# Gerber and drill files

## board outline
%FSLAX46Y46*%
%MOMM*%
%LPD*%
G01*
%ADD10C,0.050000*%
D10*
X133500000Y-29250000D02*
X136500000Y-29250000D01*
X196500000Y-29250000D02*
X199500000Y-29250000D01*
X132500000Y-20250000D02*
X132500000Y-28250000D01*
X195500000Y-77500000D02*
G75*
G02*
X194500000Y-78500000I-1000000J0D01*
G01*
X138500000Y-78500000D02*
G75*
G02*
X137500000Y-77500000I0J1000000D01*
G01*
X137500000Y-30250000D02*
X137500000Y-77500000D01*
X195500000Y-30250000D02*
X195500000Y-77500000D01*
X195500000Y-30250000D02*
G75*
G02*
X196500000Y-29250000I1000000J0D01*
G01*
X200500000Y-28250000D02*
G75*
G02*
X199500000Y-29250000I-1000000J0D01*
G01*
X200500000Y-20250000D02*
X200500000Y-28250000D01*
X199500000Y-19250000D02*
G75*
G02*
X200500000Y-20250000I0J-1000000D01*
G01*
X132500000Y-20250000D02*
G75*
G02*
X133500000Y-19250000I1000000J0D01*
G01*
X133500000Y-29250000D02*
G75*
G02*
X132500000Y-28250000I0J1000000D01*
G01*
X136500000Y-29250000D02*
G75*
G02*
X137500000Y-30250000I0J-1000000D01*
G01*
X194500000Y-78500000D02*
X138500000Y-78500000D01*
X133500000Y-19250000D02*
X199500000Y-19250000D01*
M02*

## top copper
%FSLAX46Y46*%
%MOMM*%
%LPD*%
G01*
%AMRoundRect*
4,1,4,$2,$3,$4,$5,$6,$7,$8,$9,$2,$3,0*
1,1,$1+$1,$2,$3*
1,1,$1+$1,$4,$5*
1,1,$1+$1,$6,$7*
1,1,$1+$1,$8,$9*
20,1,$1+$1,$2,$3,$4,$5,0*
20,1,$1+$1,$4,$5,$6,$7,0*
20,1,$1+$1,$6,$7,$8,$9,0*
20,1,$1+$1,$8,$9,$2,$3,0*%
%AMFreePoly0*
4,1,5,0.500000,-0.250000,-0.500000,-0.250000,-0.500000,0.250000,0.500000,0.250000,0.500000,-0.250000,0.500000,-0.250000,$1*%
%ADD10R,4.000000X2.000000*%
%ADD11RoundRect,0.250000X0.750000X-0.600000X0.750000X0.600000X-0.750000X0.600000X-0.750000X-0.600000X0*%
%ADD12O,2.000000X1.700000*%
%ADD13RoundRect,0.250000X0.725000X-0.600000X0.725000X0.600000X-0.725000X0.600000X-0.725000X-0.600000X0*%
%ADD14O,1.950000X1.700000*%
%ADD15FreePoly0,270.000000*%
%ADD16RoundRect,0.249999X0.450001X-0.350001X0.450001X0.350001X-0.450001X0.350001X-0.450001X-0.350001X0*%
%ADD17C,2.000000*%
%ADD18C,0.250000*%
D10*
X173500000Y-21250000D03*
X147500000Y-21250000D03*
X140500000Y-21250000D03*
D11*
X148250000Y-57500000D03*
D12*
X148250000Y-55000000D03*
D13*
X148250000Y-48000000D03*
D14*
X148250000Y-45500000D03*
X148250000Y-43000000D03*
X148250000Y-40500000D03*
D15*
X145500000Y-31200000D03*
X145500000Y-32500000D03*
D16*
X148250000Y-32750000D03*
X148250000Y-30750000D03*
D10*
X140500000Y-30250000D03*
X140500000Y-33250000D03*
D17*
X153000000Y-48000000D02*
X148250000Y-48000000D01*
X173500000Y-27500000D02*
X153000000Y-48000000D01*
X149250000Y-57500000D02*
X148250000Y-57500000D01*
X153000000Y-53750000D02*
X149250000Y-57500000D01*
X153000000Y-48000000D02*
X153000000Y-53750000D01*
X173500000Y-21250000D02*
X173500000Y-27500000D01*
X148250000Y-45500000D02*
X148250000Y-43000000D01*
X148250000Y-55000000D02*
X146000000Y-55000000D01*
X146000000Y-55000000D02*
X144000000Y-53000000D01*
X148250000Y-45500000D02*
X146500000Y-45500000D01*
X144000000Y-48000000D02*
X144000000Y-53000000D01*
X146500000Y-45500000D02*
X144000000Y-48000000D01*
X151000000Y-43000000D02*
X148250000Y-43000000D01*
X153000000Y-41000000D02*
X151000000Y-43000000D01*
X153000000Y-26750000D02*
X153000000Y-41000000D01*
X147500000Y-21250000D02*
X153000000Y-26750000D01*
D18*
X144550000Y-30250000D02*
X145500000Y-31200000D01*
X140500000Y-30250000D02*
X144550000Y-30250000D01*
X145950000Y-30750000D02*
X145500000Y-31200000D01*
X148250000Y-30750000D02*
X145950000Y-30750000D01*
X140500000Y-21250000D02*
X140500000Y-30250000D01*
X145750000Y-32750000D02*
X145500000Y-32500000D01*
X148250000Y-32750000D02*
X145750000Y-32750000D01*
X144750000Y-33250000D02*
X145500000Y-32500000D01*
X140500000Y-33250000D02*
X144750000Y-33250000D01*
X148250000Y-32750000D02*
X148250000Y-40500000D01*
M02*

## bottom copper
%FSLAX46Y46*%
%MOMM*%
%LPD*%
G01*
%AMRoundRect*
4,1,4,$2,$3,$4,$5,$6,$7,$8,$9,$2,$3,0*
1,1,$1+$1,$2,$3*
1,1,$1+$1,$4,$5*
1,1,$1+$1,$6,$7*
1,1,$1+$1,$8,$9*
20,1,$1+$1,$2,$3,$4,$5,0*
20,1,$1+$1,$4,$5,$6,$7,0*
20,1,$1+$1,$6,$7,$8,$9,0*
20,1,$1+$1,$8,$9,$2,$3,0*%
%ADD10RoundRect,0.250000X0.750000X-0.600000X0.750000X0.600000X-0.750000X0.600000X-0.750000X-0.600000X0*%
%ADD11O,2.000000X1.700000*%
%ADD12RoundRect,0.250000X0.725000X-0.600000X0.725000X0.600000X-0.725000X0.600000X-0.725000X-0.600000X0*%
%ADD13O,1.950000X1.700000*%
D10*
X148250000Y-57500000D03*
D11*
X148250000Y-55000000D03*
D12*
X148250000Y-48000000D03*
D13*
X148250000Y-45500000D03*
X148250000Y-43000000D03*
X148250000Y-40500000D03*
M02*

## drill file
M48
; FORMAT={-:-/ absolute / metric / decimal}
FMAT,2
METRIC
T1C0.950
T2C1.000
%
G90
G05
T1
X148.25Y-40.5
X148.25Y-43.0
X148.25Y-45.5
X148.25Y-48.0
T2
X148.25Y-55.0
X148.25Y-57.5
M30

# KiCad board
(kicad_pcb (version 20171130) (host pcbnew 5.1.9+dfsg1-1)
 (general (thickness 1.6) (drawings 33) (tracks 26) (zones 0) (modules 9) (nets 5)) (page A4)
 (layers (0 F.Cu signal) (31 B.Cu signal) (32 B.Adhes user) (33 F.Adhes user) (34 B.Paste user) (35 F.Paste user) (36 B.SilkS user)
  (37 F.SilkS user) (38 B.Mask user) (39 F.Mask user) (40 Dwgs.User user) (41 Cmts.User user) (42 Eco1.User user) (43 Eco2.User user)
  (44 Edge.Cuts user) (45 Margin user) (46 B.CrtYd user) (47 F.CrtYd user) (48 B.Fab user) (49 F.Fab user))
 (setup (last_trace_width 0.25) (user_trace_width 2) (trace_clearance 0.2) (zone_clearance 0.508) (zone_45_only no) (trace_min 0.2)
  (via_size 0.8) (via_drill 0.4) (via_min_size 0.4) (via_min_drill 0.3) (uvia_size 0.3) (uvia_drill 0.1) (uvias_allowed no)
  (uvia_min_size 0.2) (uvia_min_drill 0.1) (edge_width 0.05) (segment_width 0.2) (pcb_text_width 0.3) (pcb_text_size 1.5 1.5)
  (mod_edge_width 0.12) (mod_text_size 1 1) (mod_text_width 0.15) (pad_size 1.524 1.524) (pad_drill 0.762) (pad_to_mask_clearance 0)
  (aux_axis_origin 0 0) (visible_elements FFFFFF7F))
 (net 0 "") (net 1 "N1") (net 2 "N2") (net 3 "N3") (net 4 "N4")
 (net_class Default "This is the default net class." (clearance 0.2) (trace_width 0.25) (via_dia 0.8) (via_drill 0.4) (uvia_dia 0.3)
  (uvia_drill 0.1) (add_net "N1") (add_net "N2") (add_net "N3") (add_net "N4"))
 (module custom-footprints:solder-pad (layer F.Cu) (at 176.04 21.25 90)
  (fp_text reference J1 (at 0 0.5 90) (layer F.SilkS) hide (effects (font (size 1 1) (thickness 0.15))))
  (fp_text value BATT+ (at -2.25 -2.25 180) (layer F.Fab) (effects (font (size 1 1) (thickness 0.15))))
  (pad 1 smd rect (at 0 -2.54 90) (size 2 4) (layers F.Cu F.Paste F.Mask) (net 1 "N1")))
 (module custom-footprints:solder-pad (layer F.Cu) (at 150.04 21.25 90)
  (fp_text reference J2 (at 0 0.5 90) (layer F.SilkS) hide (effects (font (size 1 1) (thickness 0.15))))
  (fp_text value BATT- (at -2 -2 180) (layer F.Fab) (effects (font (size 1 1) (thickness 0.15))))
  (pad 1 smd rect (at 0 -2.54 90) (size 2 4) (layers F.Cu F.Paste F.Mask) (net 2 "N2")))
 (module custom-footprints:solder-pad (layer F.Cu) (at 143.04 21.25 90)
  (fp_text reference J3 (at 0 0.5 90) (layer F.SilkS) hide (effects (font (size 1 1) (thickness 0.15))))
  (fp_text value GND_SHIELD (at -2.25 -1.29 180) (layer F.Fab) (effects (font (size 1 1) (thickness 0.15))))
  (pad 1 smd rect (at 0 -2.54 90) (size 2 4) (layers F.Cu F.Paste F.Mask) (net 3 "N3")))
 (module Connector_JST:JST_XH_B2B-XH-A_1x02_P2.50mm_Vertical (layer B.Cu) (at 148.25 57.5 90)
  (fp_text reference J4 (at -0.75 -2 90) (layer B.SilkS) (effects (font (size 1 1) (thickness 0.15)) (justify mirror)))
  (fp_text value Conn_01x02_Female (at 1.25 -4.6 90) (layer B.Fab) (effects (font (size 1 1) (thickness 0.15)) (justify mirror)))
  (pad 1 thru_hole roundrect (at 0 0 90) (size 1.7 2) (drill 1) (layers *.Cu *.Mask) (roundrect_rratio 0.1470588235294118) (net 1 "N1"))
  (pad 2 thru_hole oval (at 2.5 0 90) (size 1.7 2) (drill 1) (layers *.Cu *.Mask) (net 2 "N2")))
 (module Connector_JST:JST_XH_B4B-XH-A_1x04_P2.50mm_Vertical (layer B.Cu) (at 148.25 48 90)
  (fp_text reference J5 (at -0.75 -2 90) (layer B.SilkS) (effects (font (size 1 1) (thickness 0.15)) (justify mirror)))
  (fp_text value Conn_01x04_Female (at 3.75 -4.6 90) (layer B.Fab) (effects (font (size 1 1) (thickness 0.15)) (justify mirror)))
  (pad 1 thru_hole roundrect (at 0 0 90) (size 1.7 1.95) (drill 0.95) (layers *.Cu *.Mask) (roundrect_rratio 0.1470588235294118)
   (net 1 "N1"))
  (pad 2 thru_hole oval (at 2.5 0 90) (size 1.7 1.95) (drill 0.95) (layers *.Cu *.Mask) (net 2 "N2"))
  (pad 3 thru_hole oval (at 5 0 90) (size 1.7 1.95) (drill 0.95) (layers *.Cu *.Mask) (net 2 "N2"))
  (pad 4 thru_hole oval (at 7.5 0 90) (size 1.7 1.95) (drill 0.95) (layers *.Cu *.Mask) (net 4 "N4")))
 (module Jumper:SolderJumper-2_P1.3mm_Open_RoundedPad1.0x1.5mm (layer F.Cu) (at 145.5 31.85 270)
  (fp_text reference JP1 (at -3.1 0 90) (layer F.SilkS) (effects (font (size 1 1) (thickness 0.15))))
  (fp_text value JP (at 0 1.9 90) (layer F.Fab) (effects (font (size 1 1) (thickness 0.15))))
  (pad 1 smd custom (at -0.65 0 270) (size 1 0.5) (layers F.Cu F.Mask) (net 3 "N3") (zone_connect 2)
   (options (clearance outline) (anchor rect)) (primitives))
  (pad 2 smd custom (at 0.65 0 270) (size 1 0.5) (layers F.Cu F.Mask) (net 4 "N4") (zone_connect 2)
   (options (clearance outline) (anchor rect)) (primitives)))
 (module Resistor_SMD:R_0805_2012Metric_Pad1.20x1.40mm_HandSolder (layer F.Cu) (at 148.25 31.75 90)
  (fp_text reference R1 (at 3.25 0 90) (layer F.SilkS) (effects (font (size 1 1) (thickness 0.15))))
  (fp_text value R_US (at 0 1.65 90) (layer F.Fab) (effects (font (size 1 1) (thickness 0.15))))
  (pad 1 smd roundrect (at -1 0 90) (size 1.2 1.4) (layers F.Cu F.Paste F.Mask) (roundrect_rratio 0.2083325) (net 4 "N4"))
  (pad 2 smd roundrect (at 1 0 90) (size 1.2 1.4) (layers F.Cu F.Paste F.Mask) (roundrect_rratio 0.2083325) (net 3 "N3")))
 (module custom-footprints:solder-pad (layer F.Cu) (at 143.04 30.25 90)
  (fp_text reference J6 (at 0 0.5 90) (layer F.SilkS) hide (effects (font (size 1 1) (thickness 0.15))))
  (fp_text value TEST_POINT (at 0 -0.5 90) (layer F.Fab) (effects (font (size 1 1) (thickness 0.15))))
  (pad 1 smd rect (at 0 -2.54 90) (size 2 4) (layers F.Cu F.Paste F.Mask) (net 3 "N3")))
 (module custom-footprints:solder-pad (layer F.Cu) (at 143.04 33.25 90)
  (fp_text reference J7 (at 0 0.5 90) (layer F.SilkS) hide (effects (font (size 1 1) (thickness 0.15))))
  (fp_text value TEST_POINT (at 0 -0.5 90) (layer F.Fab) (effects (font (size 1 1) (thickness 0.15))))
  (pad 1 smd rect (at 0 -2.54 90) (size 2 4) (layers F.Cu F.Paste F.Mask) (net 4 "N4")))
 (gr_line (start 133.5 29.25) (end 136.5 29.25) (layer Edge.Cuts) (width 0.05))
 (gr_line (start 196.5 29.25) (end 199.5 29.25) (layer Edge.Cuts) (width 0.05))
 (gr_line (start 132.5 20.25) (end 132.5 28.25) (layer Edge.Cuts) (width 0.05))
 (gr_arc (start 194.5 77.5) (end 194.5 78.5) (angle -90) (layer Edge.Cuts) (width 0.05))
 (gr_arc (start 138.5 77.5) (end 137.5 77.5) (angle -90) (layer Edge.Cuts) (width 0.05))
 (gr_line (start 137.5 30.25) (end 137.5 77.5) (layer Edge.Cuts) (width 0.05))
 (gr_line (start 195.5 30.25) (end 195.5 77.5) (layer Edge.Cuts) (width 0.05))
 (gr_arc (start 196.5 30.25) (end 196.5 29.25) (angle -90) (layer Edge.Cuts) (width 0.05))
 (gr_arc (start 199.5 28.25) (end 199.5 29.25) (angle -90) (layer Edge.Cuts) (width 0.05))
 (gr_line (start 200.5 20.25) (end 200.5 28.25) (layer Edge.Cuts) (width 0.05))
 (gr_arc (start 199.5 20.25) (end 200.5 20.25) (angle -90) (layer Edge.Cuts) (width 0.05))
 (gr_arc (start 133.5 20.25) (end 133.5 19.25) (angle -90) (layer Edge.Cuts) (width 0.05))
 (gr_arc (start 133.5 28.25) (end 132.5 28.25) (angle -90) (layer Edge.Cuts) (width 0.05))
 (gr_arc (start 136.5 30.25) (end 137.5 30.25) (angle -90) (layer Edge.Cuts) (width 0.05))
 (gr_line (start 194.5 78.5) (end 138.5 78.5) (layer Edge.Cuts) (width 0.05))
 (gr_line (start 133.5 19.25) (end 199.5 19.25) (layer Edge.Cuts) (width 0.05))
 (segment (start 153 48) (end 148.25 48) (width 2) (layer F.Cu) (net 1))
 (segment (start 173.5 27.5) (end 153 48) (width 2) (layer F.Cu) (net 1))
 (segment (start 149.25 57.5) (end 148.25 57.5) (width 2) (layer F.Cu) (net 1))
 (segment (start 153 53.75) (end 149.25 57.5) (width 2) (layer F.Cu) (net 1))
 (segment (start 153 48) (end 153 53.75) (width 2) (layer F.Cu) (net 1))
 (segment (start 173.5 21.25) (end 173.5 27.5) (width 2) (layer F.Cu) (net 1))
 (segment (start 148.25 45.5) (end 148.25 43) (width 2) (layer F.Cu) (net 2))
 (segment (start 148.25 55) (end 146 55) (width 2) (layer F.Cu) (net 2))
 (segment (start 146 55) (end 144 53) (width 2) (layer F.Cu) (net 2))
 (segment (start 148.25 45.5) (end 146.5 45.5) (width 2) (layer F.Cu) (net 2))
 (segment (start 144 48) (end 144 53) (width 2) (layer F.Cu) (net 2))
 (segment (start 146.5 45.5) (end 144 48) (width 2) (layer F.Cu) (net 2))
 (segment (start 151 43) (end 148.25 43) (width 2) (layer F.Cu) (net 2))
 (segment (start 153 41) (end 151 43) (width 2) (layer F.Cu) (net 2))
 (segment (start 153 26.75) (end 153 41) (width 2) (layer F.Cu) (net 2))
 (segment (start 147.5 21.25) (end 153 26.75) (width 2) (layer F.Cu) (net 2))
 (segment (start 144.55 30.25) (end 145.5 31.2) (width 0.25) (layer F.Cu) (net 3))
 (segment (start 140.5 30.25) (end 144.55 30.25) (width 0.25) (layer F.Cu) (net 3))
 (segment (start 145.95 30.75) (end 145.5 31.2) (width 0.25) (layer F.Cu) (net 3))
 (segment (start 148.25 30.75) (end 145.95 30.75) (width 0.25) (layer F.Cu) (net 3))
 (segment (start 140.5 21.25) (end 140.5 30.25) (width 0.25) (layer F.Cu) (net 3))
 (segment (start 145.75 32.75) (end 145.5 32.5) (width 0.25) (layer F.Cu) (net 4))
 (segment (start 148.25 32.75) (end 145.75 32.75) (width 0.25) (layer F.Cu) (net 4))
 (segment (start 144.75 33.25) (end 145.5 32.5) (width 0.25) (layer F.Cu) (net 4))
 (segment (start 140.5 33.25) (end 144.75 33.25) (width 0.25) (layer F.Cu) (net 4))
 (segment (start 148.25 32.75) (end 148.25 40.5) (width 0.25) (layer F.Cu) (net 4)))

